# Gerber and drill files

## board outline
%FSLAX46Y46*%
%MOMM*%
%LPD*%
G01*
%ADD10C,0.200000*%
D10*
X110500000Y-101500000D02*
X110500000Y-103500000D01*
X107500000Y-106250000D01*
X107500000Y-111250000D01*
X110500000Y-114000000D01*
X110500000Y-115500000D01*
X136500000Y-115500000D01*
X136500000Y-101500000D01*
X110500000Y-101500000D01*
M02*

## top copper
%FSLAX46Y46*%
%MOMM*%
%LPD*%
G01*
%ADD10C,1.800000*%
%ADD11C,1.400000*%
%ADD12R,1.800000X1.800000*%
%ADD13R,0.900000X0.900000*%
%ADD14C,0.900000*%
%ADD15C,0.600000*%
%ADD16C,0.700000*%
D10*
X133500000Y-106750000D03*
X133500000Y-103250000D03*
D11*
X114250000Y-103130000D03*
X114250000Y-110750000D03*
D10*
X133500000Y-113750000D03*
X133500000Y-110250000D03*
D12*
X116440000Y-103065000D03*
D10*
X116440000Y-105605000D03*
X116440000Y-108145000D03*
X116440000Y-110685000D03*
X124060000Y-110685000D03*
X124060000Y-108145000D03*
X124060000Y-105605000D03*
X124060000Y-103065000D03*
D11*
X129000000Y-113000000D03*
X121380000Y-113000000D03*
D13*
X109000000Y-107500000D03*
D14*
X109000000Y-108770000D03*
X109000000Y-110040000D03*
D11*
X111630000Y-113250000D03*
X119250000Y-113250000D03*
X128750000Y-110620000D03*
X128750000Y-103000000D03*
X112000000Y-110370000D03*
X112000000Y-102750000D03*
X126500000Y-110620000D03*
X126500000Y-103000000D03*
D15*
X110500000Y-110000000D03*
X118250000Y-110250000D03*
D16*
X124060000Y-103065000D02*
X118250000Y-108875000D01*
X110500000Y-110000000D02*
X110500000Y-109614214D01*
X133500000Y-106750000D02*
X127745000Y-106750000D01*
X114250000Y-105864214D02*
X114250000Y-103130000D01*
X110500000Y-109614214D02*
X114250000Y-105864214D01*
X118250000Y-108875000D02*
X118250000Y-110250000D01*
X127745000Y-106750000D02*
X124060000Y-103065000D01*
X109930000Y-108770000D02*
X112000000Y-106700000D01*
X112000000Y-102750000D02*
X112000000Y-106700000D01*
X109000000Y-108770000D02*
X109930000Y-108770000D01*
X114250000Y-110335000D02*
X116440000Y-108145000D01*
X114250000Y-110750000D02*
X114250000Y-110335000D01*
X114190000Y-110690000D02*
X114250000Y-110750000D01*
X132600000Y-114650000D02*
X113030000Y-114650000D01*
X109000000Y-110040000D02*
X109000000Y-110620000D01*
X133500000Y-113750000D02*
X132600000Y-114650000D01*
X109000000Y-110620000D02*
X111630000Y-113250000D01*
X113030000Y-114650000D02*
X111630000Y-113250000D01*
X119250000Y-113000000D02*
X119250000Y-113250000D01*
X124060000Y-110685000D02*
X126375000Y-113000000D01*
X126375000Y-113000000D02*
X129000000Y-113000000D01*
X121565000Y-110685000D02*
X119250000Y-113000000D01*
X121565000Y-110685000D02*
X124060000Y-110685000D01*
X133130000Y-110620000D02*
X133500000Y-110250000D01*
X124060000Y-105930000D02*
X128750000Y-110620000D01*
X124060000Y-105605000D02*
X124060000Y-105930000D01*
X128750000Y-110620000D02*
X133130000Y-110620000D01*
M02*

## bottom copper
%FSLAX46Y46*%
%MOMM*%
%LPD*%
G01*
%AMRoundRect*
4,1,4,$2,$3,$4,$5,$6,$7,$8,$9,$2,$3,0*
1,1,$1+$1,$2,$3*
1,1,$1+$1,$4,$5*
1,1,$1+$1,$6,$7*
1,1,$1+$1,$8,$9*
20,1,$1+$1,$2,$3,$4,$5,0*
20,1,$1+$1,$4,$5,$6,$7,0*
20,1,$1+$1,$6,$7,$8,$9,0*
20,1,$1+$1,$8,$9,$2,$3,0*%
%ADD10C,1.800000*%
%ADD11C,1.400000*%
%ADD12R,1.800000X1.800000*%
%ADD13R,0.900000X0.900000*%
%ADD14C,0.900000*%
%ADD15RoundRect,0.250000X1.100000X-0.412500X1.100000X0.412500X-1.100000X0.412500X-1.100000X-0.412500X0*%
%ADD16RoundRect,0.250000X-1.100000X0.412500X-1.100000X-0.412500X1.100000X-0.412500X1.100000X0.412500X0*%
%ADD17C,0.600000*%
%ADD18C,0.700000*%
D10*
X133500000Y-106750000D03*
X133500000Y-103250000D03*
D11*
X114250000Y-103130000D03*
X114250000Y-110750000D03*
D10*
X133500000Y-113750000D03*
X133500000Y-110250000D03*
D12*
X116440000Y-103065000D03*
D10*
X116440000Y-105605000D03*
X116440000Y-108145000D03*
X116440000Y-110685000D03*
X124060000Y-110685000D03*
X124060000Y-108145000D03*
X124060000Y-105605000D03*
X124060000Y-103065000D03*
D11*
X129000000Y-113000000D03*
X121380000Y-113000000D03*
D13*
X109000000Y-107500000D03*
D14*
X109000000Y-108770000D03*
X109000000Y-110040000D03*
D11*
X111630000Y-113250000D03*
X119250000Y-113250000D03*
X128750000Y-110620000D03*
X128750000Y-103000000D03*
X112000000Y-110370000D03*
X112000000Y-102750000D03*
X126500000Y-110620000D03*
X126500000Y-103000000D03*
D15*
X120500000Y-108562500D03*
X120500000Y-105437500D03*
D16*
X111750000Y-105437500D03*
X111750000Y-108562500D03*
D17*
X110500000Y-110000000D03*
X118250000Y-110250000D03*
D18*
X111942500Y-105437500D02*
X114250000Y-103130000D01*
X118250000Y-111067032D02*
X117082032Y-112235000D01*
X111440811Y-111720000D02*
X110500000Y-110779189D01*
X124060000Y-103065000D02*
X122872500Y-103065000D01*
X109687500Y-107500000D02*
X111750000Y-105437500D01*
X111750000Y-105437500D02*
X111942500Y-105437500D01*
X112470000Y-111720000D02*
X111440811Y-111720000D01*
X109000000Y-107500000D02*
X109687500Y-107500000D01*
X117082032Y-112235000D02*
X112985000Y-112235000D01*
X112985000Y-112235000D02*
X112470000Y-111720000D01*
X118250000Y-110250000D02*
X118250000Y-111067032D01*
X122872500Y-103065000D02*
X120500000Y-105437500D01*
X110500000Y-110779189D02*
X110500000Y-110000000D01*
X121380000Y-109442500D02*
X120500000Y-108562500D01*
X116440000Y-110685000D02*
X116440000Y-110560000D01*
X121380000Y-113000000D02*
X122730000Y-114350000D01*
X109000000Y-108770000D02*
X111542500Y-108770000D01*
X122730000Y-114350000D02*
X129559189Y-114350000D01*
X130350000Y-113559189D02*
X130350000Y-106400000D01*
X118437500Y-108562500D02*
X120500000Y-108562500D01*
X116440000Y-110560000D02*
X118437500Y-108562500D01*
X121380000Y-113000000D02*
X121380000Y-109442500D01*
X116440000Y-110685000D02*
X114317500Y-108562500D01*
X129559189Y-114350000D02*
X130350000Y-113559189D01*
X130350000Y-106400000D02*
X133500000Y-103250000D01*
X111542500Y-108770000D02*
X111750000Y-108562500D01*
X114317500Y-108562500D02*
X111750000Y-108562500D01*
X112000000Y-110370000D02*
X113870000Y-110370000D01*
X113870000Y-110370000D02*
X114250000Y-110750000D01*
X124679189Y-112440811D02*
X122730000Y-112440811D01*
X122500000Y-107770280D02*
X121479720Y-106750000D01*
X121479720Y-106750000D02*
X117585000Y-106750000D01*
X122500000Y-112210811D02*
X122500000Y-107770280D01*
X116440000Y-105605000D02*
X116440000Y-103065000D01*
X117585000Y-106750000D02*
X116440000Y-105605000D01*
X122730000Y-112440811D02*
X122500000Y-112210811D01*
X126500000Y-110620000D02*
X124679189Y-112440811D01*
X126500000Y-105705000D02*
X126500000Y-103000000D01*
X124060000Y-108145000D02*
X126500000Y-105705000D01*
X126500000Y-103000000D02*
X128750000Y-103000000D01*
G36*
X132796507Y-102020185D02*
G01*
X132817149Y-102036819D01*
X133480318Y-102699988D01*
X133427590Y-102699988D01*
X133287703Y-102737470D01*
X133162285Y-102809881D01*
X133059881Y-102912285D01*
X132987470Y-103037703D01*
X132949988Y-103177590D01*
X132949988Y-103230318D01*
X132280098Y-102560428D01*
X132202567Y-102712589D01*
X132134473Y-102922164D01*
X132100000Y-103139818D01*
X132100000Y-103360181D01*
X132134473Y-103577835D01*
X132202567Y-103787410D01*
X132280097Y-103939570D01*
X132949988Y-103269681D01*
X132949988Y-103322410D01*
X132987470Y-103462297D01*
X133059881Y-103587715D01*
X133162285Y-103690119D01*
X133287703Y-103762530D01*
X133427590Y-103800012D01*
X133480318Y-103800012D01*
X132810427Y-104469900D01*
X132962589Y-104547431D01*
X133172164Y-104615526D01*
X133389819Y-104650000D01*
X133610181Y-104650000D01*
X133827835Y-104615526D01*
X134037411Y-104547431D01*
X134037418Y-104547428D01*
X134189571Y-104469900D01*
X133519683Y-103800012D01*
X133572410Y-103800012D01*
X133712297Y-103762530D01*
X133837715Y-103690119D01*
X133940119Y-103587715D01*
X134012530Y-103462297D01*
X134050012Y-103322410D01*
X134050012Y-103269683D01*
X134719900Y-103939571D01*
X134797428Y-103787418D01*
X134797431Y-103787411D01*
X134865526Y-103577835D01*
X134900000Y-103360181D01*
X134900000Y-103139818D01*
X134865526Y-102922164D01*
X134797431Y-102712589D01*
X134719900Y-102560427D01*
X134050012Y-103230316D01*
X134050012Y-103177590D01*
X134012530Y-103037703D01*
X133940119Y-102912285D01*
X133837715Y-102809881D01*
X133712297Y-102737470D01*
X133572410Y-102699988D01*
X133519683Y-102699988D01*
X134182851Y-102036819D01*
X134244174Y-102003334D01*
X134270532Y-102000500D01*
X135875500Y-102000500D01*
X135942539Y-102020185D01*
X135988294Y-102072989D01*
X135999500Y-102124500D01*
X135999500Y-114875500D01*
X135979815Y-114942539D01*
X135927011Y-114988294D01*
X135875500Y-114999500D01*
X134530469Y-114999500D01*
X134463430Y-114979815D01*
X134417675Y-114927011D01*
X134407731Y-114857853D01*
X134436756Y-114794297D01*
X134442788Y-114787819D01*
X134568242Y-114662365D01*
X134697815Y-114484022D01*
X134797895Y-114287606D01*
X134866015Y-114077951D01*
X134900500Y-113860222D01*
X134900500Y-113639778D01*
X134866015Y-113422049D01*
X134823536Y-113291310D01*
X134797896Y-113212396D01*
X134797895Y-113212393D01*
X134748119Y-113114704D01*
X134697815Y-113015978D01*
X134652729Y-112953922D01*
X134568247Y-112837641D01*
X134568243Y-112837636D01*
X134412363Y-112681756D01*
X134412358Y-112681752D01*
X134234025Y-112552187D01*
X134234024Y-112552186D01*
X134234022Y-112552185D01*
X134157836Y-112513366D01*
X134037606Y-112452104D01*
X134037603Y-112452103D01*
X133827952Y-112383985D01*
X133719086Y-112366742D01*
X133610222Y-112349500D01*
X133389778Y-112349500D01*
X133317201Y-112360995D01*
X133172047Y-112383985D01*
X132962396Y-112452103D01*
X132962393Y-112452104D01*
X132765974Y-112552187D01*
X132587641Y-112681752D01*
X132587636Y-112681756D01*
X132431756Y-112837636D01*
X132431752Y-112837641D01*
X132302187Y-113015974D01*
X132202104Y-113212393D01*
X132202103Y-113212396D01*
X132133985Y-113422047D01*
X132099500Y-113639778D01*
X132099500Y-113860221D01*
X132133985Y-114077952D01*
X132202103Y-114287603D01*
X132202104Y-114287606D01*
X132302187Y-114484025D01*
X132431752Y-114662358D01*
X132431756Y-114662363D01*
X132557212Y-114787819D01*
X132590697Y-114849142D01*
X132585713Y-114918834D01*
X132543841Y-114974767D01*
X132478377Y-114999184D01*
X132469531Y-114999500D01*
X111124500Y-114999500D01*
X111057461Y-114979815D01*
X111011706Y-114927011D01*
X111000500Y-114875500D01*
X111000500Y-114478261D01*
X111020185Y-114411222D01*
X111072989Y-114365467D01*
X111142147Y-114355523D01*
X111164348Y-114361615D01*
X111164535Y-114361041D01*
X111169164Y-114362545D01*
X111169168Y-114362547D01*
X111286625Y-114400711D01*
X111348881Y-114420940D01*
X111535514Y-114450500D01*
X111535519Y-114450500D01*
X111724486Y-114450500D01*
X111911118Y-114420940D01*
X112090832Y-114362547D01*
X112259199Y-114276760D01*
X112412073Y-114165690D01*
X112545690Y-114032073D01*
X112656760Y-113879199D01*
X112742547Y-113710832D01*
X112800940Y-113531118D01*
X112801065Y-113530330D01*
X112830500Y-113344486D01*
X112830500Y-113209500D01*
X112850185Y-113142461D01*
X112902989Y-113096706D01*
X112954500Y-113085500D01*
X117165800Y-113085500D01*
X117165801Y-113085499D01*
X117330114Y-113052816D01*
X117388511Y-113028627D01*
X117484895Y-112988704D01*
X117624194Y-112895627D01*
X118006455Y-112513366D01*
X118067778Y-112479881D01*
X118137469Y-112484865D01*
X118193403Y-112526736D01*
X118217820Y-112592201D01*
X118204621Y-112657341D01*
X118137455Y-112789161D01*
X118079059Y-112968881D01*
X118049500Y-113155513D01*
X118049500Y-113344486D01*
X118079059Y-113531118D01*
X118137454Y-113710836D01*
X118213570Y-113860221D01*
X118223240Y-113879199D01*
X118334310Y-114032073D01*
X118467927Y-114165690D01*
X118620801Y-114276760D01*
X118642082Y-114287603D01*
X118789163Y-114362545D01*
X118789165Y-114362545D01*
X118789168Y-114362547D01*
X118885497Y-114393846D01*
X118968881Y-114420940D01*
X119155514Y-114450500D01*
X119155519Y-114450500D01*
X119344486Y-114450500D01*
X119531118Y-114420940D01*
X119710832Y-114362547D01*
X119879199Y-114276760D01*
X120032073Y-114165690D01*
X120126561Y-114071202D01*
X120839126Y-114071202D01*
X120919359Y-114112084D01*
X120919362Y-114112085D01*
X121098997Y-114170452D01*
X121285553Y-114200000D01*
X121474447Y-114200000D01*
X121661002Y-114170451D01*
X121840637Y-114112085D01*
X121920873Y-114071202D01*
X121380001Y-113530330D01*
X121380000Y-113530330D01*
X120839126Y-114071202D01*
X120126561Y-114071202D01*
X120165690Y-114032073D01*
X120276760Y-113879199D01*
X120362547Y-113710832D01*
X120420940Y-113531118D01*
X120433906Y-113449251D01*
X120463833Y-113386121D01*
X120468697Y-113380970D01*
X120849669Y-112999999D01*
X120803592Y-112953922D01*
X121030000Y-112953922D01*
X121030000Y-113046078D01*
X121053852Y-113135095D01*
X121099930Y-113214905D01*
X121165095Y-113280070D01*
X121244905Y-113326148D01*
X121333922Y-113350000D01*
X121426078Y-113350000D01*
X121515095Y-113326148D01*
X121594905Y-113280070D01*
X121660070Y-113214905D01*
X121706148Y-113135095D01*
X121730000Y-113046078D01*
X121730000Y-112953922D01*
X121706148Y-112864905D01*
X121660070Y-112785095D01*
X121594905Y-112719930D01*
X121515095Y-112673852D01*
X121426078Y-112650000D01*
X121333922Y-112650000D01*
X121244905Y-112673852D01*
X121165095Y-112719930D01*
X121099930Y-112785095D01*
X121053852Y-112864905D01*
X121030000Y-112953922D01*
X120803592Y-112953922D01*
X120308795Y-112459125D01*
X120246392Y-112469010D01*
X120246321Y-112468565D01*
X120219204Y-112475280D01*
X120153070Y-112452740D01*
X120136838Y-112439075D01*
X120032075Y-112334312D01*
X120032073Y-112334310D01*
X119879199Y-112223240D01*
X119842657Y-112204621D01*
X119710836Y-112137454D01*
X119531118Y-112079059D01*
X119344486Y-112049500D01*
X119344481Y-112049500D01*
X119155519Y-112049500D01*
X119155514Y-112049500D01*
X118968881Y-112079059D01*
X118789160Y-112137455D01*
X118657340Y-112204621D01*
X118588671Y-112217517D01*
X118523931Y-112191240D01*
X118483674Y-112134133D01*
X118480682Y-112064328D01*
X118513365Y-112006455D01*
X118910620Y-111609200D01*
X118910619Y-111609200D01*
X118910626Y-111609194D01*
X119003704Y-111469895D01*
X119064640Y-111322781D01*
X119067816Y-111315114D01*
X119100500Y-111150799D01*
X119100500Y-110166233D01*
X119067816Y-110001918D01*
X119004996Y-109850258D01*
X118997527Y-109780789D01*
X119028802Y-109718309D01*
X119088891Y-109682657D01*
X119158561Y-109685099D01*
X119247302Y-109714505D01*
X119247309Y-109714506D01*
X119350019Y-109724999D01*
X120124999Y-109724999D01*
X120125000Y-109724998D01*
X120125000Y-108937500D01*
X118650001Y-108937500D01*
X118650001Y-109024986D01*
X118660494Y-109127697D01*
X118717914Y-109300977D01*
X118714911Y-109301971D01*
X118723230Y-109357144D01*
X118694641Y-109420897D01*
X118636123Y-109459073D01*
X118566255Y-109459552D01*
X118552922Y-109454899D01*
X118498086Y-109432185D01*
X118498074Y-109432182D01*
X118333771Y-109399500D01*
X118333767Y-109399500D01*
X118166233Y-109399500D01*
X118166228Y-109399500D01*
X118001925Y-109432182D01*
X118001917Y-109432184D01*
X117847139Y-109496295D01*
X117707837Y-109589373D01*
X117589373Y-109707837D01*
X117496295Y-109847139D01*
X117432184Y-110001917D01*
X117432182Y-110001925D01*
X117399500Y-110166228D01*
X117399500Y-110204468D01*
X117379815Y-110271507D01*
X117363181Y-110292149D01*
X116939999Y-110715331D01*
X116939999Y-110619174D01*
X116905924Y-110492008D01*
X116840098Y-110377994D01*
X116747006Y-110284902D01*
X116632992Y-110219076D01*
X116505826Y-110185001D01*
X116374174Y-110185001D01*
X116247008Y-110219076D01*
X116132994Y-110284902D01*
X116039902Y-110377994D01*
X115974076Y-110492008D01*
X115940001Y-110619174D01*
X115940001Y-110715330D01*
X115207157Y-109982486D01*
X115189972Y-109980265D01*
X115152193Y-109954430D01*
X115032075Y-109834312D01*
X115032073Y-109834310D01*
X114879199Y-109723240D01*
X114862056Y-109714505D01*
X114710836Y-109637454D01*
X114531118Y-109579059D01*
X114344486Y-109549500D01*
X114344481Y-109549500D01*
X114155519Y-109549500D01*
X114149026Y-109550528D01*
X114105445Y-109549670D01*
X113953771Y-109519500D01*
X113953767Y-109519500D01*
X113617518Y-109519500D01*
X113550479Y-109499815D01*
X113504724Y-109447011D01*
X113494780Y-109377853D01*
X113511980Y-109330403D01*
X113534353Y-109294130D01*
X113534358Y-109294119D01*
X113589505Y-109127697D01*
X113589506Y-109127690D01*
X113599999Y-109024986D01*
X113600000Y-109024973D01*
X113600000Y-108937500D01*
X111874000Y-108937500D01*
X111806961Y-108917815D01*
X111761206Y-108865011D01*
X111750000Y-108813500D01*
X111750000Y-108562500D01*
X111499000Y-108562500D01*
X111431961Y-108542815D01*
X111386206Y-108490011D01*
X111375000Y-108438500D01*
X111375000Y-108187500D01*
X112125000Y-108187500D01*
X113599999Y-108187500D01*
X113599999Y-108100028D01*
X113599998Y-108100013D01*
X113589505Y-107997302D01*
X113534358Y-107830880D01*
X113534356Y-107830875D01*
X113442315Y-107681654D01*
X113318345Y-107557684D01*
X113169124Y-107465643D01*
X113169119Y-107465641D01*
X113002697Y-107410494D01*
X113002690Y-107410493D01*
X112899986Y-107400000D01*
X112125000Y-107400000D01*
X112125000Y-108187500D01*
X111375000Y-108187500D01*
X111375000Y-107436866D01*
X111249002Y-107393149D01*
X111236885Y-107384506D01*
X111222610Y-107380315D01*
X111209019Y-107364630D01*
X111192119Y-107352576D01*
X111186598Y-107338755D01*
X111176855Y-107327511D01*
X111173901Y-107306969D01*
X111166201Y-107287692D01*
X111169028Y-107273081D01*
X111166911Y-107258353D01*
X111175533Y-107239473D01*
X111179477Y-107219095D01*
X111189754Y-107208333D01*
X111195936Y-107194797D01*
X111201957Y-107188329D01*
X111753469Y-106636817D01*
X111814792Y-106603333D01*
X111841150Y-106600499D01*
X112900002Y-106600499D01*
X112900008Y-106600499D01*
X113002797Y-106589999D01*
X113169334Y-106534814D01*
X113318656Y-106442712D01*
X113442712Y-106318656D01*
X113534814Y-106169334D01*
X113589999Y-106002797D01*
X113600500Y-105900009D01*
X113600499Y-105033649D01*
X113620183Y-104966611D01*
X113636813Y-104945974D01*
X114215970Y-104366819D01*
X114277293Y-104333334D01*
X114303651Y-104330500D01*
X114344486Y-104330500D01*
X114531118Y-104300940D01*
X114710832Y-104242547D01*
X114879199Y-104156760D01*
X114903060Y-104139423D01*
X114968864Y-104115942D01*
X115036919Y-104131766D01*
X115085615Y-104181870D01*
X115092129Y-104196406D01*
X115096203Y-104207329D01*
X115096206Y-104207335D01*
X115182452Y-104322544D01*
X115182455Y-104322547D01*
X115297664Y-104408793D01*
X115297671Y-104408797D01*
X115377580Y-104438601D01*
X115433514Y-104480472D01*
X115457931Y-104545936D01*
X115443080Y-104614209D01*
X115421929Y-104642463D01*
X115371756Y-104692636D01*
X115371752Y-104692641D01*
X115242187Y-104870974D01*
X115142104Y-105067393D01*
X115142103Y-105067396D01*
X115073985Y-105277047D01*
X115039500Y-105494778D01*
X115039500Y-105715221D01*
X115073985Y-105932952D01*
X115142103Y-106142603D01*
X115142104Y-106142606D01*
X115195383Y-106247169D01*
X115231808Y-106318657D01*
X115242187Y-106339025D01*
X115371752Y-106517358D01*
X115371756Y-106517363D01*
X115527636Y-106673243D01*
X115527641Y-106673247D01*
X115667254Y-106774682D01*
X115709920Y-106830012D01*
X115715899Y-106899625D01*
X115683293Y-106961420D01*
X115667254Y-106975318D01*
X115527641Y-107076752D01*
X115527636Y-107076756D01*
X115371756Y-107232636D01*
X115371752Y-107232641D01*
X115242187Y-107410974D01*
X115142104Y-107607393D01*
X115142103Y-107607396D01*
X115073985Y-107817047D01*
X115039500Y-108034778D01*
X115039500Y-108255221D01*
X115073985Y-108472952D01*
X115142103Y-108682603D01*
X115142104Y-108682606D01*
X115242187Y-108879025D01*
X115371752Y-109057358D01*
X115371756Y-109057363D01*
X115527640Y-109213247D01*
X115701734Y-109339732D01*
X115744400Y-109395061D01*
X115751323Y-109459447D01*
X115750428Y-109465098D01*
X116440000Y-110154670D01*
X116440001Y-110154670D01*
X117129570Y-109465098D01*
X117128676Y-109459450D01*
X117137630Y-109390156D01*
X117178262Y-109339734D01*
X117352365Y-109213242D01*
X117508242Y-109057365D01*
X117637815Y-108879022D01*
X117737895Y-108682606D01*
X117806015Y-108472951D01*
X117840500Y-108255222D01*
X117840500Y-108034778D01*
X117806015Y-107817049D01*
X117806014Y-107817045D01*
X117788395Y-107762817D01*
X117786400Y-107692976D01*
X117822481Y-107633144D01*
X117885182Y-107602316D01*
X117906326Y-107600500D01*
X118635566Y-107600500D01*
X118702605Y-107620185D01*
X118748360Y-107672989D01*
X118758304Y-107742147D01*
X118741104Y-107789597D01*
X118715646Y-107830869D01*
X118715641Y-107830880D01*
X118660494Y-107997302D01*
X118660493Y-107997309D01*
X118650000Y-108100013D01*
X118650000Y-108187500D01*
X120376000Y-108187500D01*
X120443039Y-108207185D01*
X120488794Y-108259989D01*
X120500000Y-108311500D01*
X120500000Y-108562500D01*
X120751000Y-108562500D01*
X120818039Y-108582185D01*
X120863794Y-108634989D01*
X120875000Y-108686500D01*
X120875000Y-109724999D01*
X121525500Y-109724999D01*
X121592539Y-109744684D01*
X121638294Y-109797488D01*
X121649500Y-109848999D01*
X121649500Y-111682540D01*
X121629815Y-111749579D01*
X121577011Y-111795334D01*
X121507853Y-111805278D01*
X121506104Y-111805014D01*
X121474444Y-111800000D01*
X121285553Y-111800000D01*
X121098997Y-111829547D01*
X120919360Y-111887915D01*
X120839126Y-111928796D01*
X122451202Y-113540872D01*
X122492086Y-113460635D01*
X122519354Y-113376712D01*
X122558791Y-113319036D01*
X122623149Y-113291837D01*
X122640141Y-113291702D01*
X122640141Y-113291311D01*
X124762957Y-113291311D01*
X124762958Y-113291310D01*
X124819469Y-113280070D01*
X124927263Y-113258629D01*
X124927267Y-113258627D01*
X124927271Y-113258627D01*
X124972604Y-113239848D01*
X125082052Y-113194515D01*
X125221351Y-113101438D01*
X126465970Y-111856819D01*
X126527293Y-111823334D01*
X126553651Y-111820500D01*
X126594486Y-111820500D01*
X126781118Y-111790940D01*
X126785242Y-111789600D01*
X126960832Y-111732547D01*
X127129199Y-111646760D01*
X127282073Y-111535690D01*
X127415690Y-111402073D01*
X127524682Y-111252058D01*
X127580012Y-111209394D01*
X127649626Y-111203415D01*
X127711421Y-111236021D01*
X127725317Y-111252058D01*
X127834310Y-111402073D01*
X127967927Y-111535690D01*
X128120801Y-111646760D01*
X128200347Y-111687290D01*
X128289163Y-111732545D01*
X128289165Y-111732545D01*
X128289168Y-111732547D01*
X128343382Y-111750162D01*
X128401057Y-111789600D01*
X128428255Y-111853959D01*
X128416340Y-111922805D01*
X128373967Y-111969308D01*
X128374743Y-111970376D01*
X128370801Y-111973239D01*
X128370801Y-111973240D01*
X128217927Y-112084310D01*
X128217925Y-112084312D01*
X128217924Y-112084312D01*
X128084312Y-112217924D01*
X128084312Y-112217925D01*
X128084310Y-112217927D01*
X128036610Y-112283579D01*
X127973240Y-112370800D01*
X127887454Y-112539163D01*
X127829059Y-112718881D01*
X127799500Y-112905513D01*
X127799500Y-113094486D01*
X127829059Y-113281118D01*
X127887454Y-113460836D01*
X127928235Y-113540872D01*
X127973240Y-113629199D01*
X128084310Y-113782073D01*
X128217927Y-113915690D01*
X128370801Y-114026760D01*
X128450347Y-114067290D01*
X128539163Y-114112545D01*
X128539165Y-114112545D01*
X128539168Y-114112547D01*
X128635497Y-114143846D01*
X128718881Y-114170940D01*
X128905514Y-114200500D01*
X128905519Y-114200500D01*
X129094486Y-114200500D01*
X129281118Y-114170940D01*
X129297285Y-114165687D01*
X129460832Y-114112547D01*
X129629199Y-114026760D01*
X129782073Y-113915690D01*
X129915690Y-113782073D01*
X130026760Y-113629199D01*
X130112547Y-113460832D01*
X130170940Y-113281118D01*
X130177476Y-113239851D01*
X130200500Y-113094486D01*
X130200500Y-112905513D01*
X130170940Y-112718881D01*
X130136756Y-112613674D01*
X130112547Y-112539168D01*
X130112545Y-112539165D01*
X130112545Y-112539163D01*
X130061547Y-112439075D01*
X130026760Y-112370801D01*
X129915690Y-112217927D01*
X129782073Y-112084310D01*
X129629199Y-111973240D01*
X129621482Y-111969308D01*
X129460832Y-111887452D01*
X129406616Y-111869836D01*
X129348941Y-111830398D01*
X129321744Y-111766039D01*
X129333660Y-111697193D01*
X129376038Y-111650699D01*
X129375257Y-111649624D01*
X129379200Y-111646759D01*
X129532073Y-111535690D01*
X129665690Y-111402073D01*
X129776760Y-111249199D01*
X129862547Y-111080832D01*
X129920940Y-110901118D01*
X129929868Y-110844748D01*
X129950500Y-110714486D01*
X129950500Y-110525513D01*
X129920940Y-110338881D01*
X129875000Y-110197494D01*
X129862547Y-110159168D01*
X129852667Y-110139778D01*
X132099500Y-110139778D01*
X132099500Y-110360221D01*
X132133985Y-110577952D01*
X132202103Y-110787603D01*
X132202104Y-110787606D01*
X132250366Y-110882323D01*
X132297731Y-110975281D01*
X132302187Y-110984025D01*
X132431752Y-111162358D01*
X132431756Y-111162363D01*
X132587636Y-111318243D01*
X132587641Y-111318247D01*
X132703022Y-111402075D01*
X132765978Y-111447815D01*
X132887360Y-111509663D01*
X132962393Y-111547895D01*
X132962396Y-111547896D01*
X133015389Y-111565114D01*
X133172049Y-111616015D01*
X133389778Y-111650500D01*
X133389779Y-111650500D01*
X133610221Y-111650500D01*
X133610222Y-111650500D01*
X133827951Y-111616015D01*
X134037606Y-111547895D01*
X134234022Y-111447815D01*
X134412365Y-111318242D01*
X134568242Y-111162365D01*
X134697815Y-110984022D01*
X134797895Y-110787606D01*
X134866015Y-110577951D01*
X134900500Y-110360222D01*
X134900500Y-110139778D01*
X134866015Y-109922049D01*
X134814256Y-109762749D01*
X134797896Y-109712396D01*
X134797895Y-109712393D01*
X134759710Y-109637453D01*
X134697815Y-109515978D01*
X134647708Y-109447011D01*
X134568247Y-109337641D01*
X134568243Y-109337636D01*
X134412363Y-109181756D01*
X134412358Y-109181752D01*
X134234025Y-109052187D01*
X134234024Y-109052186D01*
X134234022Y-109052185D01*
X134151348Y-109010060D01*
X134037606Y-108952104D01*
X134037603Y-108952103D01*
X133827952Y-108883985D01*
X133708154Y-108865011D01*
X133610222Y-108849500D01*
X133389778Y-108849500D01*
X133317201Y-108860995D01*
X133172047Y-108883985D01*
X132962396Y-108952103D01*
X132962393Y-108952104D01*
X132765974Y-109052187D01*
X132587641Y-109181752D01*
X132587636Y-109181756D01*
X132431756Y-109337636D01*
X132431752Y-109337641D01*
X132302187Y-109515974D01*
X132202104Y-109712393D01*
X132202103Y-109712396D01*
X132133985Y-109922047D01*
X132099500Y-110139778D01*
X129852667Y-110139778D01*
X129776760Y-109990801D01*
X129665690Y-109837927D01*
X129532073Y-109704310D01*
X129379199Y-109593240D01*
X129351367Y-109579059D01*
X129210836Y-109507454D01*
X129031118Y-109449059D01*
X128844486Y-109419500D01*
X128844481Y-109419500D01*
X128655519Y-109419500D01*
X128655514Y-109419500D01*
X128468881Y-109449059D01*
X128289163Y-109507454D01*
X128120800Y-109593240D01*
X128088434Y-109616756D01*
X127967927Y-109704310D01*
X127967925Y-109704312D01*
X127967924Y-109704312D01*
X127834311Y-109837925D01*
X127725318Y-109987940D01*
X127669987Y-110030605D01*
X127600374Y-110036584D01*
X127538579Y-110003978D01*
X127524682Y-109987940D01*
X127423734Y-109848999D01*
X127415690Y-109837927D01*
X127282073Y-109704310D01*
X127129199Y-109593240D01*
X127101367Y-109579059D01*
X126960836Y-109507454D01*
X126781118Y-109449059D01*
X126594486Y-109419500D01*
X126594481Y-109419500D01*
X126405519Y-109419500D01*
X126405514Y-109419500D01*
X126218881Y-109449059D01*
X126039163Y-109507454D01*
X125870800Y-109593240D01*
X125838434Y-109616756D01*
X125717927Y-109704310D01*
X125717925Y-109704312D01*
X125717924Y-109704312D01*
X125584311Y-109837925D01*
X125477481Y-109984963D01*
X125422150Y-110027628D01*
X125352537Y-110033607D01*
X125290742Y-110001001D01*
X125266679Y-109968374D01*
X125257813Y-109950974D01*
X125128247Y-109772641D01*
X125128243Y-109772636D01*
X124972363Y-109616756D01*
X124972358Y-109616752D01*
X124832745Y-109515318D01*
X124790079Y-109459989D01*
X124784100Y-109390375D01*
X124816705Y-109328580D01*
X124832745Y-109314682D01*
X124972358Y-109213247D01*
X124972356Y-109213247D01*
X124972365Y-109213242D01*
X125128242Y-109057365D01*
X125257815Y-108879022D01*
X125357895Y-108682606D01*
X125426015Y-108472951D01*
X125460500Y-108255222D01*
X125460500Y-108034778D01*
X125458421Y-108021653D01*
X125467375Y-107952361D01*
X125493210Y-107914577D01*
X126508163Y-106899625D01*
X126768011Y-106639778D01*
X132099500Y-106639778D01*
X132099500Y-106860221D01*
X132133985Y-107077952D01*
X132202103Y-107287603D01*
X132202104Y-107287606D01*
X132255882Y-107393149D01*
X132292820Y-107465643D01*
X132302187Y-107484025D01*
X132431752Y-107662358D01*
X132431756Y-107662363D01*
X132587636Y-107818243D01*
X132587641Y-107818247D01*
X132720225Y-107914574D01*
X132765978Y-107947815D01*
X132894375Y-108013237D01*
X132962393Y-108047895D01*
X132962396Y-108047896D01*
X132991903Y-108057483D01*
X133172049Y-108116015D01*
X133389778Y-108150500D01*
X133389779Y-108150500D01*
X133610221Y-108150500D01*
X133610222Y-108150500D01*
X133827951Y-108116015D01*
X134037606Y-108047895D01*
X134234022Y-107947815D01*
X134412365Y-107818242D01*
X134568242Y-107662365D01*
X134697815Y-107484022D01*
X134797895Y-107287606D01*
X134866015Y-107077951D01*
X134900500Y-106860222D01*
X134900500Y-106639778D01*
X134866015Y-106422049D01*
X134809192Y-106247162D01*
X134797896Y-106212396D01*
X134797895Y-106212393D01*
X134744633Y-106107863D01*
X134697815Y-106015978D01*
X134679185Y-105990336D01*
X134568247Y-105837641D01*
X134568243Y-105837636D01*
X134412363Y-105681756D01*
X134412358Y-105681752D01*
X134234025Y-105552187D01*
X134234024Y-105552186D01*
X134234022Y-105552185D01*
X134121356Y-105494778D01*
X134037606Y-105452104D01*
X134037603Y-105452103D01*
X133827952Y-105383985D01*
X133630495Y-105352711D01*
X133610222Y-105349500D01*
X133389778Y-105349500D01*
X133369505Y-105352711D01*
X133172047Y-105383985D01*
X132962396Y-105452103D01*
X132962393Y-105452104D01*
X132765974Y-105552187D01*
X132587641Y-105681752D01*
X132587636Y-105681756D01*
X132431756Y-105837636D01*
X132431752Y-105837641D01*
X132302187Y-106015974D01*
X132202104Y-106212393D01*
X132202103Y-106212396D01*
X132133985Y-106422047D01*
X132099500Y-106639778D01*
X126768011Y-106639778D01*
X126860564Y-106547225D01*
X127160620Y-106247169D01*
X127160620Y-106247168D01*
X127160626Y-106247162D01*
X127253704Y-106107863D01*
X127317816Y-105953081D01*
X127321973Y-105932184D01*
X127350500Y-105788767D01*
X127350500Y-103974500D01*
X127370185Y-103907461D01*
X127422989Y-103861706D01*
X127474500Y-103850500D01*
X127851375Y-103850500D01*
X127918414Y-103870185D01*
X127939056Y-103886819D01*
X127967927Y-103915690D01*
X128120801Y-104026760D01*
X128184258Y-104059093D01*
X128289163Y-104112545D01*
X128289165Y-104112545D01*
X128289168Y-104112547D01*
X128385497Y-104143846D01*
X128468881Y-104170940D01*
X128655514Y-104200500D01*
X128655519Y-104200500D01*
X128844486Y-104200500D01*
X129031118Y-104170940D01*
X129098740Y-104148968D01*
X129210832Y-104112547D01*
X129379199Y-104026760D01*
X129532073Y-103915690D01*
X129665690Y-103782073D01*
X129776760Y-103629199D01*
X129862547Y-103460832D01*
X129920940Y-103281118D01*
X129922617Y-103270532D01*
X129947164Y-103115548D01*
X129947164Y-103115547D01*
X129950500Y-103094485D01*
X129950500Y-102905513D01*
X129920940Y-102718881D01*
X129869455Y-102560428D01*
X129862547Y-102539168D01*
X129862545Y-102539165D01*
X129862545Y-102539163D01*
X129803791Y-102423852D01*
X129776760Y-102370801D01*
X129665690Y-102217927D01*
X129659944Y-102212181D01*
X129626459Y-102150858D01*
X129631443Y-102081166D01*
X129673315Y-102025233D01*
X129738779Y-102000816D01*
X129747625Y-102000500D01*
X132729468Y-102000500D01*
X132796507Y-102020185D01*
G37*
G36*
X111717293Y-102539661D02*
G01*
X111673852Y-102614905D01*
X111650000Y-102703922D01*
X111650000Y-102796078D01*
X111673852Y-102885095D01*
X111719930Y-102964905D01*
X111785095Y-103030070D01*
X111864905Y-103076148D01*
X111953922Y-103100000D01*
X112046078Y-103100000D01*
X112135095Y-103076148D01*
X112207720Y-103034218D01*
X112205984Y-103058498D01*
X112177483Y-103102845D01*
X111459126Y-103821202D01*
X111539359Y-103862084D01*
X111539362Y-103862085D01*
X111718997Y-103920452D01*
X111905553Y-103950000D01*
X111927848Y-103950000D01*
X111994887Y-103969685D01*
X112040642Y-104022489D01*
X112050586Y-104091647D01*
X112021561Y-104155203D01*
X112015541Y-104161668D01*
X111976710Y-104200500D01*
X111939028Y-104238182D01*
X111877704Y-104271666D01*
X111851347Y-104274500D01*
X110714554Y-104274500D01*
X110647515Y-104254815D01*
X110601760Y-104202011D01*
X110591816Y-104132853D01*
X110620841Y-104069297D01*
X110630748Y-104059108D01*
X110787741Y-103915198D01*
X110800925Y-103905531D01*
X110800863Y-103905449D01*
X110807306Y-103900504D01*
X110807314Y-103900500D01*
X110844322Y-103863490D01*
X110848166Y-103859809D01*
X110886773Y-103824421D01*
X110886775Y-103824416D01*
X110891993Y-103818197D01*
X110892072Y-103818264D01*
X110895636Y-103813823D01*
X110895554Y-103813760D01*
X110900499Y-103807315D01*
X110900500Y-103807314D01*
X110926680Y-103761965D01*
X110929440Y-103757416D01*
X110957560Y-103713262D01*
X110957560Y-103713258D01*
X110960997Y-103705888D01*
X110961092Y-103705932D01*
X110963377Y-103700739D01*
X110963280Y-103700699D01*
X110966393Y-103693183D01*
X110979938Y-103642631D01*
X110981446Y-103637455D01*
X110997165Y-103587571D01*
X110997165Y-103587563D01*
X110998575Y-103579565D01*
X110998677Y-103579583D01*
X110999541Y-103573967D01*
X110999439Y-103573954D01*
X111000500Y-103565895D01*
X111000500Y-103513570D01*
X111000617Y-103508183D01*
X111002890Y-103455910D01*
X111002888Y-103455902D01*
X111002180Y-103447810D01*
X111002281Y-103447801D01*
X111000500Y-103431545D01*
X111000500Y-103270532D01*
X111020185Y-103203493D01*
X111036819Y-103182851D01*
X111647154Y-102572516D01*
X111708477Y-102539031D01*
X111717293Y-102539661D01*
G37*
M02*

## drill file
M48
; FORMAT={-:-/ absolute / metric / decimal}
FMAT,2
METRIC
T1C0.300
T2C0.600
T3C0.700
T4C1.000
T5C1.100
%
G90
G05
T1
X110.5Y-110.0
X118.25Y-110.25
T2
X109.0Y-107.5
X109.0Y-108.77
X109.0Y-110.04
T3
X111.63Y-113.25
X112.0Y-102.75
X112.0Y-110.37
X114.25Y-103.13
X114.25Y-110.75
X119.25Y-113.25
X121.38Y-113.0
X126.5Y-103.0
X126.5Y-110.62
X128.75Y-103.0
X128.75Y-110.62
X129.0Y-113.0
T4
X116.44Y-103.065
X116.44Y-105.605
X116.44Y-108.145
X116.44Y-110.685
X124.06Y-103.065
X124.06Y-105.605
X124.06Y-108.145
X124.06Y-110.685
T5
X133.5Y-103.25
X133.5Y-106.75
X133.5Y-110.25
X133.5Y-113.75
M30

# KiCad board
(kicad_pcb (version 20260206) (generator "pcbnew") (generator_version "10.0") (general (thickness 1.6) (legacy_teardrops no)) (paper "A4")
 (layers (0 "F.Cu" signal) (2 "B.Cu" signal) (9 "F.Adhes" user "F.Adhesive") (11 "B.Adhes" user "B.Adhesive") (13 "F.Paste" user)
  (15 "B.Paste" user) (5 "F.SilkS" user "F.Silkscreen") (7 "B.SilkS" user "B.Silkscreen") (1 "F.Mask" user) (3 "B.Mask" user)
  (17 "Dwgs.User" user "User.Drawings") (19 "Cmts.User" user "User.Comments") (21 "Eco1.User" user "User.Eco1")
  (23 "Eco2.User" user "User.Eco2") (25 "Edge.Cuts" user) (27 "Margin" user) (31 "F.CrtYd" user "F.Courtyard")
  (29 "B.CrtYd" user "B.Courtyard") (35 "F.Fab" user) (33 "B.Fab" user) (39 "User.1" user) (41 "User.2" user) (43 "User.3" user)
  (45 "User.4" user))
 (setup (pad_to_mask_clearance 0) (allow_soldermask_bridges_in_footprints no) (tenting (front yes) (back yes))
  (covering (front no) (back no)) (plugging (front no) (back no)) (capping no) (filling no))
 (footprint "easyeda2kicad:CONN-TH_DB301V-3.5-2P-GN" (layer "F.Cu") (at 133.5 105 90)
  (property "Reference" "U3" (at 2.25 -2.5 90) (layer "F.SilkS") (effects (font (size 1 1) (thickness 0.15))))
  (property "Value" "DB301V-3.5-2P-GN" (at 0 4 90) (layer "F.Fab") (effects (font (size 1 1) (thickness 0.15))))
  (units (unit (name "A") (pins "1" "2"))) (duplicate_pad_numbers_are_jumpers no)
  (pad "1" thru_hole circle (at -1.75 0 90) (size 1.8 1.8) (drill 1.100023) (layers "*.Cu" "*.Mask") (remove_unused_layers no) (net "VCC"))
  (pad "2" thru_hole circle (at 1.75 0 90) (size 1.8 1.8) (drill 1.100023) (layers "*.Cu" "*.Mask") (remove_unused_layers no) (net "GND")))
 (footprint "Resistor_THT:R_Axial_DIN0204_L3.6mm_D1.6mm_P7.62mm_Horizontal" (layer "F.Cu") (at 114.25 103.13 -90)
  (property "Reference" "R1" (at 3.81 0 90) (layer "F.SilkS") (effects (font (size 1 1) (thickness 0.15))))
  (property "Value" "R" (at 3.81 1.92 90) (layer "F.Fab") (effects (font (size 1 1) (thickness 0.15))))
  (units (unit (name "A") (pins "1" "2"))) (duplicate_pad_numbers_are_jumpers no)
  (pad "1" thru_hole circle (at 0 0 270) (size 1.4 1.4) (drill 0.7) (layers "*.Cu" "*.Mask") (remove_unused_layers no) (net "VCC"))
  (pad "2" thru_hole circle (at 7.62 0 270) (size 1.4 1.4) (drill 0.7) (layers "*.Cu" "*.Mask") (remove_unused_layers no)
   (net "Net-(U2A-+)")))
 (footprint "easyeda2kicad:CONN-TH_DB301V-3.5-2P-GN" (layer "F.Cu") (at 133.5 112 90)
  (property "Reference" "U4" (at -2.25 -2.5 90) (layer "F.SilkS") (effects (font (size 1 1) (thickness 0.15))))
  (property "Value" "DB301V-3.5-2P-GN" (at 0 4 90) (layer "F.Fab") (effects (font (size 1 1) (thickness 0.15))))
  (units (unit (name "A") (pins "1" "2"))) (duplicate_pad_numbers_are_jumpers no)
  (pad "1" thru_hole circle (at -1.75 0 90) (size 1.8 1.8) (drill 1.100023) (layers "*.Cu" "*.Mask") (remove_unused_layers no)
   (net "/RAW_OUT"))
  (pad "2" thru_hole circle (at 1.75 0 90) (size 1.8 1.8) (drill 1.100023) (layers "*.Cu" "*.Mask") (remove_unused_layers no) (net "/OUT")))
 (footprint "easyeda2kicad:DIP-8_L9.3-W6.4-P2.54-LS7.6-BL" (layer "F.Cu") (at 120.25 106.875 -90)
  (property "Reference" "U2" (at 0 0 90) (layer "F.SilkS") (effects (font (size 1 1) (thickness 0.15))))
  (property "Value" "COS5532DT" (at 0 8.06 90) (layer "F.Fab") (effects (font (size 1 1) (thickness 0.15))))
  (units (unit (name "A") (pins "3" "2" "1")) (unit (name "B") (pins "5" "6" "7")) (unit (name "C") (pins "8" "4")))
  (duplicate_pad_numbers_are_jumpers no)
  (pad "1" thru_hole rect (at -3.81 3.81 270) (size 1.8 1.8) (drill 0.999998) (layers "*.Cu" "*.Mask") (remove_unused_layers no)
   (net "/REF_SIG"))
  (pad "2" thru_hole circle (at -1.27 3.81 270) (size 1.8 1.8) (drill 0.999998) (layers "*.Cu" "*.Mask") (remove_unused_layers no)
   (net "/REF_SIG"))
  (pad "3" thru_hole circle (at 1.27 3.81 270) (size 1.8 1.8) (drill 0.999998) (layers "*.Cu" "*.Mask") (remove_unused_layers no)
   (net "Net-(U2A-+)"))
  (pad "4" thru_hole circle (at 3.81 3.81 270) (size 1.8 1.8) (drill 0.999998) (layers "*.Cu" "*.Mask") (remove_unused_layers no)
   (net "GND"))
  (pad "5" thru_hole circle (at 3.81 -3.81 270) (size 1.8 1.8) (drill 0.999998) (layers "*.Cu" "*.Mask") (remove_unused_layers no)
   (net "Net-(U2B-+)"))
  (pad "6" thru_hole circle (at 1.27 -3.81 270) (size 1.8 1.8) (drill 0.999998) (layers "*.Cu" "*.Mask") (remove_unused_layers no)
   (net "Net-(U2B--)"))
  (pad "7" thru_hole circle (at -1.27 -3.81 270) (size 1.8 1.8) (drill 0.999998) (layers "*.Cu" "*.Mask") (remove_unused_layers no)
   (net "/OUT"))
  (pad "8" thru_hole circle (at -3.81 -3.81 270) (size 1.8 1.8) (drill 0.999998) (layers "*.Cu" "*.Mask") (remove_unused_layers no)
   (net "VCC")))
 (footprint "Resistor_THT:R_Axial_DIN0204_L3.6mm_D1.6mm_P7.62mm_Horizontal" (layer "F.Cu") (at 129 113 180)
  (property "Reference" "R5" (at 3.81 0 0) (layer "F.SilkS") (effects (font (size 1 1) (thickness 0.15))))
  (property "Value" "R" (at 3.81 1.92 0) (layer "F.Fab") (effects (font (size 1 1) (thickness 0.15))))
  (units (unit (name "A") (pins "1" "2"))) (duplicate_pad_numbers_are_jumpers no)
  (pad "1" thru_hole circle (at 0 0 180) (size 1.4 1.4) (drill 0.7) (layers "*.Cu" "*.Mask") (remove_unused_layers no) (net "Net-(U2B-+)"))
  (pad "2" thru_hole circle (at 7.62 0 180) (size 1.4 1.4) (drill 0.7) (layers "*.Cu" "*.Mask") (remove_unused_layers no) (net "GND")))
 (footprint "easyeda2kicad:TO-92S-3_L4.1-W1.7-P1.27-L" (layer "F.Cu") (at 109 108.77 -90)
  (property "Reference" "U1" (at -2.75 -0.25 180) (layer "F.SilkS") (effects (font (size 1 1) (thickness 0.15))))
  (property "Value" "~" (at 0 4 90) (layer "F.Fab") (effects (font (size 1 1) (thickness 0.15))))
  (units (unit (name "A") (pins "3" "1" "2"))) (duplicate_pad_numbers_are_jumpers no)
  (pad "1" thru_hole rect (at -1.27 0 270) (size 0.9 0.9) (drill 0.599999) (layers "*.Cu" "*.Mask") (remove_unused_layers no) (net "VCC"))
  (pad "2" thru_hole circle (at 0 0 270) (size 0.9 0.9) (drill 0.599999) (layers "*.Cu" "*.Mask") (remove_unused_layers no) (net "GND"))
  (pad "3" thru_hole circle (at 1.27 0 270) (size 0.9 0.9) (drill 0.599999) (layers "*.Cu" "*.Mask") (remove_unused_layers no)
   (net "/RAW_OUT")))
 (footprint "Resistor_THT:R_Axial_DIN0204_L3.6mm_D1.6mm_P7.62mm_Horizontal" (layer "F.Cu") (at 111.63 113.25)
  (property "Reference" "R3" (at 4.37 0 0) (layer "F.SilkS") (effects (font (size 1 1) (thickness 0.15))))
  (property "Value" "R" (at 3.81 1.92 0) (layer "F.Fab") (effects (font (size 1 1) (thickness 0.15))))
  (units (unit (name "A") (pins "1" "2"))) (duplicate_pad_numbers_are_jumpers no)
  (pad "1" thru_hole circle (at 0 0) (size 1.4 1.4) (drill 0.7) (layers "*.Cu" "*.Mask") (remove_unused_layers no) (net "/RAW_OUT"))
  (pad "2" thru_hole circle (at 7.62 0) (size 1.4 1.4) (drill 0.7) (layers "*.Cu" "*.Mask") (remove_unused_layers no) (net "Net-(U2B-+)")))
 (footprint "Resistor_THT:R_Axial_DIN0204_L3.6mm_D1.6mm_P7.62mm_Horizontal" (layer "F.Cu") (at 128.75 110.62 90)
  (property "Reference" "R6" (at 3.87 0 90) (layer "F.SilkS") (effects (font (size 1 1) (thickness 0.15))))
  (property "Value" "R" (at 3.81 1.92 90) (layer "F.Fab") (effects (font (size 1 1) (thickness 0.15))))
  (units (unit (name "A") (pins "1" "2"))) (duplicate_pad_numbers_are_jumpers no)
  (pad "1" thru_hole circle (at 0 0 90) (size 1.4 1.4) (drill 0.7) (layers "*.Cu" "*.Mask") (remove_unused_layers no) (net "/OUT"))
  (pad "2" thru_hole circle (at 7.62 0 90) (size 1.4 1.4) (drill 0.7) (layers "*.Cu" "*.Mask") (remove_unused_layers no) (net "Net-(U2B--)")))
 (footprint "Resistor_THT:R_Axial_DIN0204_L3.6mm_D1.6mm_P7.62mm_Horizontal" (layer "F.Cu") (at 112 110.37 90)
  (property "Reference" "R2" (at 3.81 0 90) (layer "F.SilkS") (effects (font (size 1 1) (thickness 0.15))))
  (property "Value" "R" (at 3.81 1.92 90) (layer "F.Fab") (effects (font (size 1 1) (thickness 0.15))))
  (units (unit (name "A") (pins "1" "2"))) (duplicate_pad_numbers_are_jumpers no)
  (pad "1" thru_hole circle (at 0 0 90) (size 1.4 1.4) (drill 0.7) (layers "*.Cu" "*.Mask") (remove_unused_layers no) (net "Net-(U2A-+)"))
  (pad "2" thru_hole circle (at 7.62 0 90) (size 1.4 1.4) (drill 0.7) (layers "*.Cu" "*.Mask") (remove_unused_layers no) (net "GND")))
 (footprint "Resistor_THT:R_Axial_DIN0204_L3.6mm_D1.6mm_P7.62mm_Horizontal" (layer "F.Cu") (at 126.5 110.62 90)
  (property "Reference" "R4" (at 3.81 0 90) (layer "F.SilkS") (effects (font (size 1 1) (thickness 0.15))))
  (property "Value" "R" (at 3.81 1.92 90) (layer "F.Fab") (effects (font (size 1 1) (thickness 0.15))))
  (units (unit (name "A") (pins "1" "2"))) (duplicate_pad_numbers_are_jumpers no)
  (pad "1" thru_hole circle (at 0 0 90) (size 1.4 1.4) (drill 0.7) (layers "*.Cu" "*.Mask") (remove_unused_layers no) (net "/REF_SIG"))
  (pad "2" thru_hole circle (at 7.62 0 90) (size 1.4 1.4) (drill 0.7) (layers "*.Cu" "*.Mask") (remove_unused_layers no) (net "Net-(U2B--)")))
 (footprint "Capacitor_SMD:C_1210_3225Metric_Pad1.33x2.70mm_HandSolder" (layer "B.Cu") (at 120.5 107 90)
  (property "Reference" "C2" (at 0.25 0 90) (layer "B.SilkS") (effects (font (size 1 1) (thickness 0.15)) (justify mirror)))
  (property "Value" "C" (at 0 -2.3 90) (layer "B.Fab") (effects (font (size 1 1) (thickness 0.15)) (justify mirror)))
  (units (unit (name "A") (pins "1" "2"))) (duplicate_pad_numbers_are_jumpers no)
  (pad "1" smd roundrect (at -1.5625 0 90) (size 1.325 2.7) (layers "B.Cu" "B.Mask" "B.Paste") (roundrect_rratio 0.188679) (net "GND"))
  (pad "2" smd roundrect (at 1.5625 0 90) (size 1.325 2.7) (layers "B.Cu" "B.Mask" "B.Paste") (roundrect_rratio 0.188679) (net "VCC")))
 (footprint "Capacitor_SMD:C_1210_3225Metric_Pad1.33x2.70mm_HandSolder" (layer "B.Cu") (at 111.75 107 -90)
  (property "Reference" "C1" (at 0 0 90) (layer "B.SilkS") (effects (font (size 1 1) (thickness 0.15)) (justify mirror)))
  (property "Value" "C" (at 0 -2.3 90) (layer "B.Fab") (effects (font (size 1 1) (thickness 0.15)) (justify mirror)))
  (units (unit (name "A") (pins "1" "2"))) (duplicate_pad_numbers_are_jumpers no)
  (pad "1" smd roundrect (at -1.5625 0 270) (size 1.325 2.7) (layers "B.Cu" "B.Mask" "B.Paste") (roundrect_rratio 0.188679) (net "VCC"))
  (pad "2" smd roundrect (at 1.5625 0 270) (size 1.325 2.7) (layers "B.Cu" "B.Mask" "B.Paste") (roundrect_rratio 0.188679) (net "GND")))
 (gr_poly
  (pts (xy 110.5 101.5) (xy 110.5 103.5) (xy 107.5 106.25) (xy 107.5 111.25) (xy 110.5 114) (xy 110.5 115.5) (xy 136.5 115.5)
   (xy 136.5 101.5))
  (stroke (width 0.2) (type solid)) (fill no) (layer "Edge.Cuts"))
 (segment (start 124.06 103.065) (end 118.25 108.875) (width 0.7) (layer "F.Cu") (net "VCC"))
 (segment (start 110.5 110) (end 110.5 109.614214) (width 0.7) (layer "F.Cu") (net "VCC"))
 (segment (start 133.5 106.75) (end 127.745 106.75) (width 0.7) (layer "F.Cu") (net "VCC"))
 (segment (start 114.25 105.864214) (end 114.25 103.13) (width 0.7) (layer "F.Cu") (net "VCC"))
 (segment (start 110.5 109.614214) (end 114.25 105.864214) (width 0.7) (layer "F.Cu") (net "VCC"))
 (segment (start 118.25 108.875) (end 118.25 110.25) (width 0.7) (layer "F.Cu") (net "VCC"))
 (segment (start 127.745 106.75) (end 124.06 103.065) (width 0.7) (layer "F.Cu") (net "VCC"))
 (via (at 110.5 110) (size 0.6) (drill 0.3) (layers "F.Cu" "B.Cu") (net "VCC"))
 (via (at 118.25 110.25) (size 0.6) (drill 0.3) (layers "F.Cu" "B.Cu") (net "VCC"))
 (segment (start 111.9425 105.4375) (end 114.25 103.13) (width 0.7) (layer "B.Cu") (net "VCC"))
 (segment (start 118.25 111.067032) (end 117.082032 112.235) (width 0.7) (layer "B.Cu") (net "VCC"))
 (segment (start 111.440811 111.72) (end 110.5 110.779189) (width 0.7) (layer "B.Cu") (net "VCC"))
 (segment (start 124.06 103.065) (end 122.8725 103.065) (width 0.7) (layer "B.Cu") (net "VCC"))
 (segment (start 109.6875 107.5) (end 111.75 105.4375) (width 0.7) (layer "B.Cu") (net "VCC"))
 (segment (start 111.75 105.4375) (end 111.9425 105.4375) (width 0.7) (layer "B.Cu") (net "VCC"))
 (segment (start 112.47 111.72) (end 111.440811 111.72) (width 0.7) (layer "B.Cu") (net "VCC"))
 (segment (start 109 107.5) (end 109.6875 107.5) (width 0.7) (layer "B.Cu") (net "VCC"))
 (segment (start 117.082032 112.235) (end 112.985 112.235) (width 0.7) (layer "B.Cu") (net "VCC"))
 (segment (start 112.985 112.235) (end 112.47 111.72) (width 0.7) (layer "B.Cu") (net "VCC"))
 (segment (start 118.25 110.25) (end 118.25 111.067032) (width 0.7) (layer "B.Cu") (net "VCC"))
 (segment (start 122.8725 103.065) (end 120.5 105.4375) (width 0.7) (layer "B.Cu") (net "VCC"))
 (segment (start 110.5 110.779189) (end 110.5 110) (width 0.7) (layer "B.Cu") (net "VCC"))
 (segment (start 109.93 108.77) (end 112 106.7) (width 0.7) (layer "F.Cu") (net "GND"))
 (segment (start 112 102.75) (end 112 106.7) (width 0.7) (layer "F.Cu") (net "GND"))
 (segment (start 109 108.77) (end 109.93 108.77) (width 0.7) (layer "F.Cu") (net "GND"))
 (segment (start 121.38 109.4425) (end 120.5 108.5625) (width 0.7) (layer "B.Cu") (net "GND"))
 (segment (start 116.44 110.685) (end 116.44 110.56) (width 0.7) (layer "B.Cu") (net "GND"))
 (segment (start 121.38 113) (end 122.73 114.35) (width 0.7) (layer "B.Cu") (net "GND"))
 (segment (start 109 108.77) (end 111.5425 108.77) (width 0.7) (layer "B.Cu") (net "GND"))
 (segment (start 122.73 114.35) (end 129.559189 114.35) (width 0.7) (layer "B.Cu") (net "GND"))
 (segment (start 130.35 113.559189) (end 130.35 106.4) (width 0.7) (layer "B.Cu") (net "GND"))
 (segment (start 118.4375 108.5625) (end 120.5 108.5625) (width 0.7) (layer "B.Cu") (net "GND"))
 (segment (start 116.44 110.56) (end 118.4375 108.5625) (width 0.7) (layer "B.Cu") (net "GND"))
 (segment (start 121.38 113) (end 121.38 109.4425) (width 0.7) (layer "B.Cu") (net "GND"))
 (segment (start 116.44 110.685) (end 114.3175 108.5625) (width 0.7) (layer "B.Cu") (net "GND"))
 (segment (start 129.559189 114.35) (end 130.35 113.559189) (width 0.7) (layer "B.Cu") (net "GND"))
 (segment (start 130.35 106.4) (end 133.5 103.25) (width 0.7) (layer "B.Cu") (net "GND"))
 (segment (start 111.5425 108.77) (end 111.75 108.5625) (width 0.7) (layer "B.Cu") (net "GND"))
 (segment (start 114.3175 108.5625) (end 111.75 108.5625) (width 0.7) (layer "B.Cu") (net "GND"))
 (segment (start 114.25 110.335) (end 116.44 108.145) (width 0.7) (layer "F.Cu") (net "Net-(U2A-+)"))
 (segment (start 114.25 110.75) (end 114.25 110.335) (width 0.7) (layer "F.Cu") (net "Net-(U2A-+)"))
 (segment (start 114.19 110.69) (end 114.25 110.75) (width 0.7) (layer "F.Cu") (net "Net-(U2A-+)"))
 (segment (start 112 110.37) (end 113.87 110.37) (width 0.7) (layer "B.Cu") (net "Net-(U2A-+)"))
 (segment (start 113.87 110.37) (end 114.25 110.75) (width 0.7) (layer "B.Cu") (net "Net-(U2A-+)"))
 (segment (start 132.6 114.65) (end 113.03 114.65) (width 0.7) (layer "F.Cu") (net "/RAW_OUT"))
 (segment (start 109 110.04) (end 109 110.62) (width 0.7) (layer "F.Cu") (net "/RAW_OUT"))
 (segment (start 133.5 113.75) (end 132.6 114.65) (width 0.7) (layer "F.Cu") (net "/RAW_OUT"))
 (segment (start 109 110.62) (end 111.63 113.25) (width 0.7) (layer "F.Cu") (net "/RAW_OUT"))
 (segment (start 113.03 114.65) (end 111.63 113.25) (width 0.7) (layer "F.Cu") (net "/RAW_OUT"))
 (segment (start 119.25 113) (end 119.25 113.25) (width 0.7) (layer "F.Cu") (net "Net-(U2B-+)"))
 (segment (start 124.06 110.685) (end 126.375 113) (width 0.7) (layer "F.Cu") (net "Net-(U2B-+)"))
 (segment (start 126.375 113) (end 129 113) (width 0.7) (layer "F.Cu") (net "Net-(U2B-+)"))
 (segment (start 121.565 110.685) (end 119.25 113) (width 0.7) (layer "F.Cu") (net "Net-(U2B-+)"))
 (segment (start 121.565 110.685) (end 124.06 110.685) (width 0.7) (layer "F.Cu") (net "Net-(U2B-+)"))
 (segment (start 124.679189 112.440811) (end 122.73 112.440811) (width 0.7) (layer "B.Cu") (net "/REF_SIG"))
 (segment (start 122.5 107.77028) (end 121.47972 106.75) (width 0.7) (layer "B.Cu") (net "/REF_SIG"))
 (segment (start 121.47972 106.75) (end 117.585 106.75) (width 0.7) (layer "B.Cu") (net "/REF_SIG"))
 (segment (start 122.5 112.210811) (end 122.5 107.77028) (width 0.7) (layer "B.Cu") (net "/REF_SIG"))
 (segment (start 116.44 105.605) (end 116.44 103.065) (width 0.7) (layer "B.Cu") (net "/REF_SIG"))
 (segment (start 117.585 106.75) (end 116.44 105.605) (width 0.7) (layer "B.Cu") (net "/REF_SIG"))
 (segment (start 122.73 112.440811) (end 122.5 112.210811) (width 0.7) (layer "B.Cu") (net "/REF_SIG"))
 (segment (start 126.5 110.62) (end 124.679189 112.440811) (width 0.7) (layer "B.Cu") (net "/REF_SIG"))
 (segment (start 126.5 105.705) (end 126.5 103) (width 0.7) (layer "B.Cu") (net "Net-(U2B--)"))
 (segment (start 124.06 108.145) (end 126.5 105.705) (width 0.7) (layer "B.Cu") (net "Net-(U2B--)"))
 (segment (start 126.5 103) (end 128.75 103) (width 0.7) (layer "B.Cu") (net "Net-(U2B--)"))
 (segment (start 133.13 110.62) (end 133.5 110.25) (width 0.7) (layer "F.Cu") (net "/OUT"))
 (segment (start 124.06 105.93) (end 128.75 110.62) (width 0.7) (layer "F.Cu") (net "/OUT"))
 (segment (start 124.06 105.605) (end 124.06 105.93) (width 0.7) (layer "F.Cu") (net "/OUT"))
 (segment (start 128.75 110.62) (end 133.13 110.62) (width 0.7) (layer "F.Cu") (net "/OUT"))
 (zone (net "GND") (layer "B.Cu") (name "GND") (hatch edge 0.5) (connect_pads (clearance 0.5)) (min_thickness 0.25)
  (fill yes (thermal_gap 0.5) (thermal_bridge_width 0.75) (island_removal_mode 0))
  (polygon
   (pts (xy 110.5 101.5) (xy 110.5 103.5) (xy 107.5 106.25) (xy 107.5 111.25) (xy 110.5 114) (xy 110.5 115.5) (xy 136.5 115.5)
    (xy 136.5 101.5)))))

